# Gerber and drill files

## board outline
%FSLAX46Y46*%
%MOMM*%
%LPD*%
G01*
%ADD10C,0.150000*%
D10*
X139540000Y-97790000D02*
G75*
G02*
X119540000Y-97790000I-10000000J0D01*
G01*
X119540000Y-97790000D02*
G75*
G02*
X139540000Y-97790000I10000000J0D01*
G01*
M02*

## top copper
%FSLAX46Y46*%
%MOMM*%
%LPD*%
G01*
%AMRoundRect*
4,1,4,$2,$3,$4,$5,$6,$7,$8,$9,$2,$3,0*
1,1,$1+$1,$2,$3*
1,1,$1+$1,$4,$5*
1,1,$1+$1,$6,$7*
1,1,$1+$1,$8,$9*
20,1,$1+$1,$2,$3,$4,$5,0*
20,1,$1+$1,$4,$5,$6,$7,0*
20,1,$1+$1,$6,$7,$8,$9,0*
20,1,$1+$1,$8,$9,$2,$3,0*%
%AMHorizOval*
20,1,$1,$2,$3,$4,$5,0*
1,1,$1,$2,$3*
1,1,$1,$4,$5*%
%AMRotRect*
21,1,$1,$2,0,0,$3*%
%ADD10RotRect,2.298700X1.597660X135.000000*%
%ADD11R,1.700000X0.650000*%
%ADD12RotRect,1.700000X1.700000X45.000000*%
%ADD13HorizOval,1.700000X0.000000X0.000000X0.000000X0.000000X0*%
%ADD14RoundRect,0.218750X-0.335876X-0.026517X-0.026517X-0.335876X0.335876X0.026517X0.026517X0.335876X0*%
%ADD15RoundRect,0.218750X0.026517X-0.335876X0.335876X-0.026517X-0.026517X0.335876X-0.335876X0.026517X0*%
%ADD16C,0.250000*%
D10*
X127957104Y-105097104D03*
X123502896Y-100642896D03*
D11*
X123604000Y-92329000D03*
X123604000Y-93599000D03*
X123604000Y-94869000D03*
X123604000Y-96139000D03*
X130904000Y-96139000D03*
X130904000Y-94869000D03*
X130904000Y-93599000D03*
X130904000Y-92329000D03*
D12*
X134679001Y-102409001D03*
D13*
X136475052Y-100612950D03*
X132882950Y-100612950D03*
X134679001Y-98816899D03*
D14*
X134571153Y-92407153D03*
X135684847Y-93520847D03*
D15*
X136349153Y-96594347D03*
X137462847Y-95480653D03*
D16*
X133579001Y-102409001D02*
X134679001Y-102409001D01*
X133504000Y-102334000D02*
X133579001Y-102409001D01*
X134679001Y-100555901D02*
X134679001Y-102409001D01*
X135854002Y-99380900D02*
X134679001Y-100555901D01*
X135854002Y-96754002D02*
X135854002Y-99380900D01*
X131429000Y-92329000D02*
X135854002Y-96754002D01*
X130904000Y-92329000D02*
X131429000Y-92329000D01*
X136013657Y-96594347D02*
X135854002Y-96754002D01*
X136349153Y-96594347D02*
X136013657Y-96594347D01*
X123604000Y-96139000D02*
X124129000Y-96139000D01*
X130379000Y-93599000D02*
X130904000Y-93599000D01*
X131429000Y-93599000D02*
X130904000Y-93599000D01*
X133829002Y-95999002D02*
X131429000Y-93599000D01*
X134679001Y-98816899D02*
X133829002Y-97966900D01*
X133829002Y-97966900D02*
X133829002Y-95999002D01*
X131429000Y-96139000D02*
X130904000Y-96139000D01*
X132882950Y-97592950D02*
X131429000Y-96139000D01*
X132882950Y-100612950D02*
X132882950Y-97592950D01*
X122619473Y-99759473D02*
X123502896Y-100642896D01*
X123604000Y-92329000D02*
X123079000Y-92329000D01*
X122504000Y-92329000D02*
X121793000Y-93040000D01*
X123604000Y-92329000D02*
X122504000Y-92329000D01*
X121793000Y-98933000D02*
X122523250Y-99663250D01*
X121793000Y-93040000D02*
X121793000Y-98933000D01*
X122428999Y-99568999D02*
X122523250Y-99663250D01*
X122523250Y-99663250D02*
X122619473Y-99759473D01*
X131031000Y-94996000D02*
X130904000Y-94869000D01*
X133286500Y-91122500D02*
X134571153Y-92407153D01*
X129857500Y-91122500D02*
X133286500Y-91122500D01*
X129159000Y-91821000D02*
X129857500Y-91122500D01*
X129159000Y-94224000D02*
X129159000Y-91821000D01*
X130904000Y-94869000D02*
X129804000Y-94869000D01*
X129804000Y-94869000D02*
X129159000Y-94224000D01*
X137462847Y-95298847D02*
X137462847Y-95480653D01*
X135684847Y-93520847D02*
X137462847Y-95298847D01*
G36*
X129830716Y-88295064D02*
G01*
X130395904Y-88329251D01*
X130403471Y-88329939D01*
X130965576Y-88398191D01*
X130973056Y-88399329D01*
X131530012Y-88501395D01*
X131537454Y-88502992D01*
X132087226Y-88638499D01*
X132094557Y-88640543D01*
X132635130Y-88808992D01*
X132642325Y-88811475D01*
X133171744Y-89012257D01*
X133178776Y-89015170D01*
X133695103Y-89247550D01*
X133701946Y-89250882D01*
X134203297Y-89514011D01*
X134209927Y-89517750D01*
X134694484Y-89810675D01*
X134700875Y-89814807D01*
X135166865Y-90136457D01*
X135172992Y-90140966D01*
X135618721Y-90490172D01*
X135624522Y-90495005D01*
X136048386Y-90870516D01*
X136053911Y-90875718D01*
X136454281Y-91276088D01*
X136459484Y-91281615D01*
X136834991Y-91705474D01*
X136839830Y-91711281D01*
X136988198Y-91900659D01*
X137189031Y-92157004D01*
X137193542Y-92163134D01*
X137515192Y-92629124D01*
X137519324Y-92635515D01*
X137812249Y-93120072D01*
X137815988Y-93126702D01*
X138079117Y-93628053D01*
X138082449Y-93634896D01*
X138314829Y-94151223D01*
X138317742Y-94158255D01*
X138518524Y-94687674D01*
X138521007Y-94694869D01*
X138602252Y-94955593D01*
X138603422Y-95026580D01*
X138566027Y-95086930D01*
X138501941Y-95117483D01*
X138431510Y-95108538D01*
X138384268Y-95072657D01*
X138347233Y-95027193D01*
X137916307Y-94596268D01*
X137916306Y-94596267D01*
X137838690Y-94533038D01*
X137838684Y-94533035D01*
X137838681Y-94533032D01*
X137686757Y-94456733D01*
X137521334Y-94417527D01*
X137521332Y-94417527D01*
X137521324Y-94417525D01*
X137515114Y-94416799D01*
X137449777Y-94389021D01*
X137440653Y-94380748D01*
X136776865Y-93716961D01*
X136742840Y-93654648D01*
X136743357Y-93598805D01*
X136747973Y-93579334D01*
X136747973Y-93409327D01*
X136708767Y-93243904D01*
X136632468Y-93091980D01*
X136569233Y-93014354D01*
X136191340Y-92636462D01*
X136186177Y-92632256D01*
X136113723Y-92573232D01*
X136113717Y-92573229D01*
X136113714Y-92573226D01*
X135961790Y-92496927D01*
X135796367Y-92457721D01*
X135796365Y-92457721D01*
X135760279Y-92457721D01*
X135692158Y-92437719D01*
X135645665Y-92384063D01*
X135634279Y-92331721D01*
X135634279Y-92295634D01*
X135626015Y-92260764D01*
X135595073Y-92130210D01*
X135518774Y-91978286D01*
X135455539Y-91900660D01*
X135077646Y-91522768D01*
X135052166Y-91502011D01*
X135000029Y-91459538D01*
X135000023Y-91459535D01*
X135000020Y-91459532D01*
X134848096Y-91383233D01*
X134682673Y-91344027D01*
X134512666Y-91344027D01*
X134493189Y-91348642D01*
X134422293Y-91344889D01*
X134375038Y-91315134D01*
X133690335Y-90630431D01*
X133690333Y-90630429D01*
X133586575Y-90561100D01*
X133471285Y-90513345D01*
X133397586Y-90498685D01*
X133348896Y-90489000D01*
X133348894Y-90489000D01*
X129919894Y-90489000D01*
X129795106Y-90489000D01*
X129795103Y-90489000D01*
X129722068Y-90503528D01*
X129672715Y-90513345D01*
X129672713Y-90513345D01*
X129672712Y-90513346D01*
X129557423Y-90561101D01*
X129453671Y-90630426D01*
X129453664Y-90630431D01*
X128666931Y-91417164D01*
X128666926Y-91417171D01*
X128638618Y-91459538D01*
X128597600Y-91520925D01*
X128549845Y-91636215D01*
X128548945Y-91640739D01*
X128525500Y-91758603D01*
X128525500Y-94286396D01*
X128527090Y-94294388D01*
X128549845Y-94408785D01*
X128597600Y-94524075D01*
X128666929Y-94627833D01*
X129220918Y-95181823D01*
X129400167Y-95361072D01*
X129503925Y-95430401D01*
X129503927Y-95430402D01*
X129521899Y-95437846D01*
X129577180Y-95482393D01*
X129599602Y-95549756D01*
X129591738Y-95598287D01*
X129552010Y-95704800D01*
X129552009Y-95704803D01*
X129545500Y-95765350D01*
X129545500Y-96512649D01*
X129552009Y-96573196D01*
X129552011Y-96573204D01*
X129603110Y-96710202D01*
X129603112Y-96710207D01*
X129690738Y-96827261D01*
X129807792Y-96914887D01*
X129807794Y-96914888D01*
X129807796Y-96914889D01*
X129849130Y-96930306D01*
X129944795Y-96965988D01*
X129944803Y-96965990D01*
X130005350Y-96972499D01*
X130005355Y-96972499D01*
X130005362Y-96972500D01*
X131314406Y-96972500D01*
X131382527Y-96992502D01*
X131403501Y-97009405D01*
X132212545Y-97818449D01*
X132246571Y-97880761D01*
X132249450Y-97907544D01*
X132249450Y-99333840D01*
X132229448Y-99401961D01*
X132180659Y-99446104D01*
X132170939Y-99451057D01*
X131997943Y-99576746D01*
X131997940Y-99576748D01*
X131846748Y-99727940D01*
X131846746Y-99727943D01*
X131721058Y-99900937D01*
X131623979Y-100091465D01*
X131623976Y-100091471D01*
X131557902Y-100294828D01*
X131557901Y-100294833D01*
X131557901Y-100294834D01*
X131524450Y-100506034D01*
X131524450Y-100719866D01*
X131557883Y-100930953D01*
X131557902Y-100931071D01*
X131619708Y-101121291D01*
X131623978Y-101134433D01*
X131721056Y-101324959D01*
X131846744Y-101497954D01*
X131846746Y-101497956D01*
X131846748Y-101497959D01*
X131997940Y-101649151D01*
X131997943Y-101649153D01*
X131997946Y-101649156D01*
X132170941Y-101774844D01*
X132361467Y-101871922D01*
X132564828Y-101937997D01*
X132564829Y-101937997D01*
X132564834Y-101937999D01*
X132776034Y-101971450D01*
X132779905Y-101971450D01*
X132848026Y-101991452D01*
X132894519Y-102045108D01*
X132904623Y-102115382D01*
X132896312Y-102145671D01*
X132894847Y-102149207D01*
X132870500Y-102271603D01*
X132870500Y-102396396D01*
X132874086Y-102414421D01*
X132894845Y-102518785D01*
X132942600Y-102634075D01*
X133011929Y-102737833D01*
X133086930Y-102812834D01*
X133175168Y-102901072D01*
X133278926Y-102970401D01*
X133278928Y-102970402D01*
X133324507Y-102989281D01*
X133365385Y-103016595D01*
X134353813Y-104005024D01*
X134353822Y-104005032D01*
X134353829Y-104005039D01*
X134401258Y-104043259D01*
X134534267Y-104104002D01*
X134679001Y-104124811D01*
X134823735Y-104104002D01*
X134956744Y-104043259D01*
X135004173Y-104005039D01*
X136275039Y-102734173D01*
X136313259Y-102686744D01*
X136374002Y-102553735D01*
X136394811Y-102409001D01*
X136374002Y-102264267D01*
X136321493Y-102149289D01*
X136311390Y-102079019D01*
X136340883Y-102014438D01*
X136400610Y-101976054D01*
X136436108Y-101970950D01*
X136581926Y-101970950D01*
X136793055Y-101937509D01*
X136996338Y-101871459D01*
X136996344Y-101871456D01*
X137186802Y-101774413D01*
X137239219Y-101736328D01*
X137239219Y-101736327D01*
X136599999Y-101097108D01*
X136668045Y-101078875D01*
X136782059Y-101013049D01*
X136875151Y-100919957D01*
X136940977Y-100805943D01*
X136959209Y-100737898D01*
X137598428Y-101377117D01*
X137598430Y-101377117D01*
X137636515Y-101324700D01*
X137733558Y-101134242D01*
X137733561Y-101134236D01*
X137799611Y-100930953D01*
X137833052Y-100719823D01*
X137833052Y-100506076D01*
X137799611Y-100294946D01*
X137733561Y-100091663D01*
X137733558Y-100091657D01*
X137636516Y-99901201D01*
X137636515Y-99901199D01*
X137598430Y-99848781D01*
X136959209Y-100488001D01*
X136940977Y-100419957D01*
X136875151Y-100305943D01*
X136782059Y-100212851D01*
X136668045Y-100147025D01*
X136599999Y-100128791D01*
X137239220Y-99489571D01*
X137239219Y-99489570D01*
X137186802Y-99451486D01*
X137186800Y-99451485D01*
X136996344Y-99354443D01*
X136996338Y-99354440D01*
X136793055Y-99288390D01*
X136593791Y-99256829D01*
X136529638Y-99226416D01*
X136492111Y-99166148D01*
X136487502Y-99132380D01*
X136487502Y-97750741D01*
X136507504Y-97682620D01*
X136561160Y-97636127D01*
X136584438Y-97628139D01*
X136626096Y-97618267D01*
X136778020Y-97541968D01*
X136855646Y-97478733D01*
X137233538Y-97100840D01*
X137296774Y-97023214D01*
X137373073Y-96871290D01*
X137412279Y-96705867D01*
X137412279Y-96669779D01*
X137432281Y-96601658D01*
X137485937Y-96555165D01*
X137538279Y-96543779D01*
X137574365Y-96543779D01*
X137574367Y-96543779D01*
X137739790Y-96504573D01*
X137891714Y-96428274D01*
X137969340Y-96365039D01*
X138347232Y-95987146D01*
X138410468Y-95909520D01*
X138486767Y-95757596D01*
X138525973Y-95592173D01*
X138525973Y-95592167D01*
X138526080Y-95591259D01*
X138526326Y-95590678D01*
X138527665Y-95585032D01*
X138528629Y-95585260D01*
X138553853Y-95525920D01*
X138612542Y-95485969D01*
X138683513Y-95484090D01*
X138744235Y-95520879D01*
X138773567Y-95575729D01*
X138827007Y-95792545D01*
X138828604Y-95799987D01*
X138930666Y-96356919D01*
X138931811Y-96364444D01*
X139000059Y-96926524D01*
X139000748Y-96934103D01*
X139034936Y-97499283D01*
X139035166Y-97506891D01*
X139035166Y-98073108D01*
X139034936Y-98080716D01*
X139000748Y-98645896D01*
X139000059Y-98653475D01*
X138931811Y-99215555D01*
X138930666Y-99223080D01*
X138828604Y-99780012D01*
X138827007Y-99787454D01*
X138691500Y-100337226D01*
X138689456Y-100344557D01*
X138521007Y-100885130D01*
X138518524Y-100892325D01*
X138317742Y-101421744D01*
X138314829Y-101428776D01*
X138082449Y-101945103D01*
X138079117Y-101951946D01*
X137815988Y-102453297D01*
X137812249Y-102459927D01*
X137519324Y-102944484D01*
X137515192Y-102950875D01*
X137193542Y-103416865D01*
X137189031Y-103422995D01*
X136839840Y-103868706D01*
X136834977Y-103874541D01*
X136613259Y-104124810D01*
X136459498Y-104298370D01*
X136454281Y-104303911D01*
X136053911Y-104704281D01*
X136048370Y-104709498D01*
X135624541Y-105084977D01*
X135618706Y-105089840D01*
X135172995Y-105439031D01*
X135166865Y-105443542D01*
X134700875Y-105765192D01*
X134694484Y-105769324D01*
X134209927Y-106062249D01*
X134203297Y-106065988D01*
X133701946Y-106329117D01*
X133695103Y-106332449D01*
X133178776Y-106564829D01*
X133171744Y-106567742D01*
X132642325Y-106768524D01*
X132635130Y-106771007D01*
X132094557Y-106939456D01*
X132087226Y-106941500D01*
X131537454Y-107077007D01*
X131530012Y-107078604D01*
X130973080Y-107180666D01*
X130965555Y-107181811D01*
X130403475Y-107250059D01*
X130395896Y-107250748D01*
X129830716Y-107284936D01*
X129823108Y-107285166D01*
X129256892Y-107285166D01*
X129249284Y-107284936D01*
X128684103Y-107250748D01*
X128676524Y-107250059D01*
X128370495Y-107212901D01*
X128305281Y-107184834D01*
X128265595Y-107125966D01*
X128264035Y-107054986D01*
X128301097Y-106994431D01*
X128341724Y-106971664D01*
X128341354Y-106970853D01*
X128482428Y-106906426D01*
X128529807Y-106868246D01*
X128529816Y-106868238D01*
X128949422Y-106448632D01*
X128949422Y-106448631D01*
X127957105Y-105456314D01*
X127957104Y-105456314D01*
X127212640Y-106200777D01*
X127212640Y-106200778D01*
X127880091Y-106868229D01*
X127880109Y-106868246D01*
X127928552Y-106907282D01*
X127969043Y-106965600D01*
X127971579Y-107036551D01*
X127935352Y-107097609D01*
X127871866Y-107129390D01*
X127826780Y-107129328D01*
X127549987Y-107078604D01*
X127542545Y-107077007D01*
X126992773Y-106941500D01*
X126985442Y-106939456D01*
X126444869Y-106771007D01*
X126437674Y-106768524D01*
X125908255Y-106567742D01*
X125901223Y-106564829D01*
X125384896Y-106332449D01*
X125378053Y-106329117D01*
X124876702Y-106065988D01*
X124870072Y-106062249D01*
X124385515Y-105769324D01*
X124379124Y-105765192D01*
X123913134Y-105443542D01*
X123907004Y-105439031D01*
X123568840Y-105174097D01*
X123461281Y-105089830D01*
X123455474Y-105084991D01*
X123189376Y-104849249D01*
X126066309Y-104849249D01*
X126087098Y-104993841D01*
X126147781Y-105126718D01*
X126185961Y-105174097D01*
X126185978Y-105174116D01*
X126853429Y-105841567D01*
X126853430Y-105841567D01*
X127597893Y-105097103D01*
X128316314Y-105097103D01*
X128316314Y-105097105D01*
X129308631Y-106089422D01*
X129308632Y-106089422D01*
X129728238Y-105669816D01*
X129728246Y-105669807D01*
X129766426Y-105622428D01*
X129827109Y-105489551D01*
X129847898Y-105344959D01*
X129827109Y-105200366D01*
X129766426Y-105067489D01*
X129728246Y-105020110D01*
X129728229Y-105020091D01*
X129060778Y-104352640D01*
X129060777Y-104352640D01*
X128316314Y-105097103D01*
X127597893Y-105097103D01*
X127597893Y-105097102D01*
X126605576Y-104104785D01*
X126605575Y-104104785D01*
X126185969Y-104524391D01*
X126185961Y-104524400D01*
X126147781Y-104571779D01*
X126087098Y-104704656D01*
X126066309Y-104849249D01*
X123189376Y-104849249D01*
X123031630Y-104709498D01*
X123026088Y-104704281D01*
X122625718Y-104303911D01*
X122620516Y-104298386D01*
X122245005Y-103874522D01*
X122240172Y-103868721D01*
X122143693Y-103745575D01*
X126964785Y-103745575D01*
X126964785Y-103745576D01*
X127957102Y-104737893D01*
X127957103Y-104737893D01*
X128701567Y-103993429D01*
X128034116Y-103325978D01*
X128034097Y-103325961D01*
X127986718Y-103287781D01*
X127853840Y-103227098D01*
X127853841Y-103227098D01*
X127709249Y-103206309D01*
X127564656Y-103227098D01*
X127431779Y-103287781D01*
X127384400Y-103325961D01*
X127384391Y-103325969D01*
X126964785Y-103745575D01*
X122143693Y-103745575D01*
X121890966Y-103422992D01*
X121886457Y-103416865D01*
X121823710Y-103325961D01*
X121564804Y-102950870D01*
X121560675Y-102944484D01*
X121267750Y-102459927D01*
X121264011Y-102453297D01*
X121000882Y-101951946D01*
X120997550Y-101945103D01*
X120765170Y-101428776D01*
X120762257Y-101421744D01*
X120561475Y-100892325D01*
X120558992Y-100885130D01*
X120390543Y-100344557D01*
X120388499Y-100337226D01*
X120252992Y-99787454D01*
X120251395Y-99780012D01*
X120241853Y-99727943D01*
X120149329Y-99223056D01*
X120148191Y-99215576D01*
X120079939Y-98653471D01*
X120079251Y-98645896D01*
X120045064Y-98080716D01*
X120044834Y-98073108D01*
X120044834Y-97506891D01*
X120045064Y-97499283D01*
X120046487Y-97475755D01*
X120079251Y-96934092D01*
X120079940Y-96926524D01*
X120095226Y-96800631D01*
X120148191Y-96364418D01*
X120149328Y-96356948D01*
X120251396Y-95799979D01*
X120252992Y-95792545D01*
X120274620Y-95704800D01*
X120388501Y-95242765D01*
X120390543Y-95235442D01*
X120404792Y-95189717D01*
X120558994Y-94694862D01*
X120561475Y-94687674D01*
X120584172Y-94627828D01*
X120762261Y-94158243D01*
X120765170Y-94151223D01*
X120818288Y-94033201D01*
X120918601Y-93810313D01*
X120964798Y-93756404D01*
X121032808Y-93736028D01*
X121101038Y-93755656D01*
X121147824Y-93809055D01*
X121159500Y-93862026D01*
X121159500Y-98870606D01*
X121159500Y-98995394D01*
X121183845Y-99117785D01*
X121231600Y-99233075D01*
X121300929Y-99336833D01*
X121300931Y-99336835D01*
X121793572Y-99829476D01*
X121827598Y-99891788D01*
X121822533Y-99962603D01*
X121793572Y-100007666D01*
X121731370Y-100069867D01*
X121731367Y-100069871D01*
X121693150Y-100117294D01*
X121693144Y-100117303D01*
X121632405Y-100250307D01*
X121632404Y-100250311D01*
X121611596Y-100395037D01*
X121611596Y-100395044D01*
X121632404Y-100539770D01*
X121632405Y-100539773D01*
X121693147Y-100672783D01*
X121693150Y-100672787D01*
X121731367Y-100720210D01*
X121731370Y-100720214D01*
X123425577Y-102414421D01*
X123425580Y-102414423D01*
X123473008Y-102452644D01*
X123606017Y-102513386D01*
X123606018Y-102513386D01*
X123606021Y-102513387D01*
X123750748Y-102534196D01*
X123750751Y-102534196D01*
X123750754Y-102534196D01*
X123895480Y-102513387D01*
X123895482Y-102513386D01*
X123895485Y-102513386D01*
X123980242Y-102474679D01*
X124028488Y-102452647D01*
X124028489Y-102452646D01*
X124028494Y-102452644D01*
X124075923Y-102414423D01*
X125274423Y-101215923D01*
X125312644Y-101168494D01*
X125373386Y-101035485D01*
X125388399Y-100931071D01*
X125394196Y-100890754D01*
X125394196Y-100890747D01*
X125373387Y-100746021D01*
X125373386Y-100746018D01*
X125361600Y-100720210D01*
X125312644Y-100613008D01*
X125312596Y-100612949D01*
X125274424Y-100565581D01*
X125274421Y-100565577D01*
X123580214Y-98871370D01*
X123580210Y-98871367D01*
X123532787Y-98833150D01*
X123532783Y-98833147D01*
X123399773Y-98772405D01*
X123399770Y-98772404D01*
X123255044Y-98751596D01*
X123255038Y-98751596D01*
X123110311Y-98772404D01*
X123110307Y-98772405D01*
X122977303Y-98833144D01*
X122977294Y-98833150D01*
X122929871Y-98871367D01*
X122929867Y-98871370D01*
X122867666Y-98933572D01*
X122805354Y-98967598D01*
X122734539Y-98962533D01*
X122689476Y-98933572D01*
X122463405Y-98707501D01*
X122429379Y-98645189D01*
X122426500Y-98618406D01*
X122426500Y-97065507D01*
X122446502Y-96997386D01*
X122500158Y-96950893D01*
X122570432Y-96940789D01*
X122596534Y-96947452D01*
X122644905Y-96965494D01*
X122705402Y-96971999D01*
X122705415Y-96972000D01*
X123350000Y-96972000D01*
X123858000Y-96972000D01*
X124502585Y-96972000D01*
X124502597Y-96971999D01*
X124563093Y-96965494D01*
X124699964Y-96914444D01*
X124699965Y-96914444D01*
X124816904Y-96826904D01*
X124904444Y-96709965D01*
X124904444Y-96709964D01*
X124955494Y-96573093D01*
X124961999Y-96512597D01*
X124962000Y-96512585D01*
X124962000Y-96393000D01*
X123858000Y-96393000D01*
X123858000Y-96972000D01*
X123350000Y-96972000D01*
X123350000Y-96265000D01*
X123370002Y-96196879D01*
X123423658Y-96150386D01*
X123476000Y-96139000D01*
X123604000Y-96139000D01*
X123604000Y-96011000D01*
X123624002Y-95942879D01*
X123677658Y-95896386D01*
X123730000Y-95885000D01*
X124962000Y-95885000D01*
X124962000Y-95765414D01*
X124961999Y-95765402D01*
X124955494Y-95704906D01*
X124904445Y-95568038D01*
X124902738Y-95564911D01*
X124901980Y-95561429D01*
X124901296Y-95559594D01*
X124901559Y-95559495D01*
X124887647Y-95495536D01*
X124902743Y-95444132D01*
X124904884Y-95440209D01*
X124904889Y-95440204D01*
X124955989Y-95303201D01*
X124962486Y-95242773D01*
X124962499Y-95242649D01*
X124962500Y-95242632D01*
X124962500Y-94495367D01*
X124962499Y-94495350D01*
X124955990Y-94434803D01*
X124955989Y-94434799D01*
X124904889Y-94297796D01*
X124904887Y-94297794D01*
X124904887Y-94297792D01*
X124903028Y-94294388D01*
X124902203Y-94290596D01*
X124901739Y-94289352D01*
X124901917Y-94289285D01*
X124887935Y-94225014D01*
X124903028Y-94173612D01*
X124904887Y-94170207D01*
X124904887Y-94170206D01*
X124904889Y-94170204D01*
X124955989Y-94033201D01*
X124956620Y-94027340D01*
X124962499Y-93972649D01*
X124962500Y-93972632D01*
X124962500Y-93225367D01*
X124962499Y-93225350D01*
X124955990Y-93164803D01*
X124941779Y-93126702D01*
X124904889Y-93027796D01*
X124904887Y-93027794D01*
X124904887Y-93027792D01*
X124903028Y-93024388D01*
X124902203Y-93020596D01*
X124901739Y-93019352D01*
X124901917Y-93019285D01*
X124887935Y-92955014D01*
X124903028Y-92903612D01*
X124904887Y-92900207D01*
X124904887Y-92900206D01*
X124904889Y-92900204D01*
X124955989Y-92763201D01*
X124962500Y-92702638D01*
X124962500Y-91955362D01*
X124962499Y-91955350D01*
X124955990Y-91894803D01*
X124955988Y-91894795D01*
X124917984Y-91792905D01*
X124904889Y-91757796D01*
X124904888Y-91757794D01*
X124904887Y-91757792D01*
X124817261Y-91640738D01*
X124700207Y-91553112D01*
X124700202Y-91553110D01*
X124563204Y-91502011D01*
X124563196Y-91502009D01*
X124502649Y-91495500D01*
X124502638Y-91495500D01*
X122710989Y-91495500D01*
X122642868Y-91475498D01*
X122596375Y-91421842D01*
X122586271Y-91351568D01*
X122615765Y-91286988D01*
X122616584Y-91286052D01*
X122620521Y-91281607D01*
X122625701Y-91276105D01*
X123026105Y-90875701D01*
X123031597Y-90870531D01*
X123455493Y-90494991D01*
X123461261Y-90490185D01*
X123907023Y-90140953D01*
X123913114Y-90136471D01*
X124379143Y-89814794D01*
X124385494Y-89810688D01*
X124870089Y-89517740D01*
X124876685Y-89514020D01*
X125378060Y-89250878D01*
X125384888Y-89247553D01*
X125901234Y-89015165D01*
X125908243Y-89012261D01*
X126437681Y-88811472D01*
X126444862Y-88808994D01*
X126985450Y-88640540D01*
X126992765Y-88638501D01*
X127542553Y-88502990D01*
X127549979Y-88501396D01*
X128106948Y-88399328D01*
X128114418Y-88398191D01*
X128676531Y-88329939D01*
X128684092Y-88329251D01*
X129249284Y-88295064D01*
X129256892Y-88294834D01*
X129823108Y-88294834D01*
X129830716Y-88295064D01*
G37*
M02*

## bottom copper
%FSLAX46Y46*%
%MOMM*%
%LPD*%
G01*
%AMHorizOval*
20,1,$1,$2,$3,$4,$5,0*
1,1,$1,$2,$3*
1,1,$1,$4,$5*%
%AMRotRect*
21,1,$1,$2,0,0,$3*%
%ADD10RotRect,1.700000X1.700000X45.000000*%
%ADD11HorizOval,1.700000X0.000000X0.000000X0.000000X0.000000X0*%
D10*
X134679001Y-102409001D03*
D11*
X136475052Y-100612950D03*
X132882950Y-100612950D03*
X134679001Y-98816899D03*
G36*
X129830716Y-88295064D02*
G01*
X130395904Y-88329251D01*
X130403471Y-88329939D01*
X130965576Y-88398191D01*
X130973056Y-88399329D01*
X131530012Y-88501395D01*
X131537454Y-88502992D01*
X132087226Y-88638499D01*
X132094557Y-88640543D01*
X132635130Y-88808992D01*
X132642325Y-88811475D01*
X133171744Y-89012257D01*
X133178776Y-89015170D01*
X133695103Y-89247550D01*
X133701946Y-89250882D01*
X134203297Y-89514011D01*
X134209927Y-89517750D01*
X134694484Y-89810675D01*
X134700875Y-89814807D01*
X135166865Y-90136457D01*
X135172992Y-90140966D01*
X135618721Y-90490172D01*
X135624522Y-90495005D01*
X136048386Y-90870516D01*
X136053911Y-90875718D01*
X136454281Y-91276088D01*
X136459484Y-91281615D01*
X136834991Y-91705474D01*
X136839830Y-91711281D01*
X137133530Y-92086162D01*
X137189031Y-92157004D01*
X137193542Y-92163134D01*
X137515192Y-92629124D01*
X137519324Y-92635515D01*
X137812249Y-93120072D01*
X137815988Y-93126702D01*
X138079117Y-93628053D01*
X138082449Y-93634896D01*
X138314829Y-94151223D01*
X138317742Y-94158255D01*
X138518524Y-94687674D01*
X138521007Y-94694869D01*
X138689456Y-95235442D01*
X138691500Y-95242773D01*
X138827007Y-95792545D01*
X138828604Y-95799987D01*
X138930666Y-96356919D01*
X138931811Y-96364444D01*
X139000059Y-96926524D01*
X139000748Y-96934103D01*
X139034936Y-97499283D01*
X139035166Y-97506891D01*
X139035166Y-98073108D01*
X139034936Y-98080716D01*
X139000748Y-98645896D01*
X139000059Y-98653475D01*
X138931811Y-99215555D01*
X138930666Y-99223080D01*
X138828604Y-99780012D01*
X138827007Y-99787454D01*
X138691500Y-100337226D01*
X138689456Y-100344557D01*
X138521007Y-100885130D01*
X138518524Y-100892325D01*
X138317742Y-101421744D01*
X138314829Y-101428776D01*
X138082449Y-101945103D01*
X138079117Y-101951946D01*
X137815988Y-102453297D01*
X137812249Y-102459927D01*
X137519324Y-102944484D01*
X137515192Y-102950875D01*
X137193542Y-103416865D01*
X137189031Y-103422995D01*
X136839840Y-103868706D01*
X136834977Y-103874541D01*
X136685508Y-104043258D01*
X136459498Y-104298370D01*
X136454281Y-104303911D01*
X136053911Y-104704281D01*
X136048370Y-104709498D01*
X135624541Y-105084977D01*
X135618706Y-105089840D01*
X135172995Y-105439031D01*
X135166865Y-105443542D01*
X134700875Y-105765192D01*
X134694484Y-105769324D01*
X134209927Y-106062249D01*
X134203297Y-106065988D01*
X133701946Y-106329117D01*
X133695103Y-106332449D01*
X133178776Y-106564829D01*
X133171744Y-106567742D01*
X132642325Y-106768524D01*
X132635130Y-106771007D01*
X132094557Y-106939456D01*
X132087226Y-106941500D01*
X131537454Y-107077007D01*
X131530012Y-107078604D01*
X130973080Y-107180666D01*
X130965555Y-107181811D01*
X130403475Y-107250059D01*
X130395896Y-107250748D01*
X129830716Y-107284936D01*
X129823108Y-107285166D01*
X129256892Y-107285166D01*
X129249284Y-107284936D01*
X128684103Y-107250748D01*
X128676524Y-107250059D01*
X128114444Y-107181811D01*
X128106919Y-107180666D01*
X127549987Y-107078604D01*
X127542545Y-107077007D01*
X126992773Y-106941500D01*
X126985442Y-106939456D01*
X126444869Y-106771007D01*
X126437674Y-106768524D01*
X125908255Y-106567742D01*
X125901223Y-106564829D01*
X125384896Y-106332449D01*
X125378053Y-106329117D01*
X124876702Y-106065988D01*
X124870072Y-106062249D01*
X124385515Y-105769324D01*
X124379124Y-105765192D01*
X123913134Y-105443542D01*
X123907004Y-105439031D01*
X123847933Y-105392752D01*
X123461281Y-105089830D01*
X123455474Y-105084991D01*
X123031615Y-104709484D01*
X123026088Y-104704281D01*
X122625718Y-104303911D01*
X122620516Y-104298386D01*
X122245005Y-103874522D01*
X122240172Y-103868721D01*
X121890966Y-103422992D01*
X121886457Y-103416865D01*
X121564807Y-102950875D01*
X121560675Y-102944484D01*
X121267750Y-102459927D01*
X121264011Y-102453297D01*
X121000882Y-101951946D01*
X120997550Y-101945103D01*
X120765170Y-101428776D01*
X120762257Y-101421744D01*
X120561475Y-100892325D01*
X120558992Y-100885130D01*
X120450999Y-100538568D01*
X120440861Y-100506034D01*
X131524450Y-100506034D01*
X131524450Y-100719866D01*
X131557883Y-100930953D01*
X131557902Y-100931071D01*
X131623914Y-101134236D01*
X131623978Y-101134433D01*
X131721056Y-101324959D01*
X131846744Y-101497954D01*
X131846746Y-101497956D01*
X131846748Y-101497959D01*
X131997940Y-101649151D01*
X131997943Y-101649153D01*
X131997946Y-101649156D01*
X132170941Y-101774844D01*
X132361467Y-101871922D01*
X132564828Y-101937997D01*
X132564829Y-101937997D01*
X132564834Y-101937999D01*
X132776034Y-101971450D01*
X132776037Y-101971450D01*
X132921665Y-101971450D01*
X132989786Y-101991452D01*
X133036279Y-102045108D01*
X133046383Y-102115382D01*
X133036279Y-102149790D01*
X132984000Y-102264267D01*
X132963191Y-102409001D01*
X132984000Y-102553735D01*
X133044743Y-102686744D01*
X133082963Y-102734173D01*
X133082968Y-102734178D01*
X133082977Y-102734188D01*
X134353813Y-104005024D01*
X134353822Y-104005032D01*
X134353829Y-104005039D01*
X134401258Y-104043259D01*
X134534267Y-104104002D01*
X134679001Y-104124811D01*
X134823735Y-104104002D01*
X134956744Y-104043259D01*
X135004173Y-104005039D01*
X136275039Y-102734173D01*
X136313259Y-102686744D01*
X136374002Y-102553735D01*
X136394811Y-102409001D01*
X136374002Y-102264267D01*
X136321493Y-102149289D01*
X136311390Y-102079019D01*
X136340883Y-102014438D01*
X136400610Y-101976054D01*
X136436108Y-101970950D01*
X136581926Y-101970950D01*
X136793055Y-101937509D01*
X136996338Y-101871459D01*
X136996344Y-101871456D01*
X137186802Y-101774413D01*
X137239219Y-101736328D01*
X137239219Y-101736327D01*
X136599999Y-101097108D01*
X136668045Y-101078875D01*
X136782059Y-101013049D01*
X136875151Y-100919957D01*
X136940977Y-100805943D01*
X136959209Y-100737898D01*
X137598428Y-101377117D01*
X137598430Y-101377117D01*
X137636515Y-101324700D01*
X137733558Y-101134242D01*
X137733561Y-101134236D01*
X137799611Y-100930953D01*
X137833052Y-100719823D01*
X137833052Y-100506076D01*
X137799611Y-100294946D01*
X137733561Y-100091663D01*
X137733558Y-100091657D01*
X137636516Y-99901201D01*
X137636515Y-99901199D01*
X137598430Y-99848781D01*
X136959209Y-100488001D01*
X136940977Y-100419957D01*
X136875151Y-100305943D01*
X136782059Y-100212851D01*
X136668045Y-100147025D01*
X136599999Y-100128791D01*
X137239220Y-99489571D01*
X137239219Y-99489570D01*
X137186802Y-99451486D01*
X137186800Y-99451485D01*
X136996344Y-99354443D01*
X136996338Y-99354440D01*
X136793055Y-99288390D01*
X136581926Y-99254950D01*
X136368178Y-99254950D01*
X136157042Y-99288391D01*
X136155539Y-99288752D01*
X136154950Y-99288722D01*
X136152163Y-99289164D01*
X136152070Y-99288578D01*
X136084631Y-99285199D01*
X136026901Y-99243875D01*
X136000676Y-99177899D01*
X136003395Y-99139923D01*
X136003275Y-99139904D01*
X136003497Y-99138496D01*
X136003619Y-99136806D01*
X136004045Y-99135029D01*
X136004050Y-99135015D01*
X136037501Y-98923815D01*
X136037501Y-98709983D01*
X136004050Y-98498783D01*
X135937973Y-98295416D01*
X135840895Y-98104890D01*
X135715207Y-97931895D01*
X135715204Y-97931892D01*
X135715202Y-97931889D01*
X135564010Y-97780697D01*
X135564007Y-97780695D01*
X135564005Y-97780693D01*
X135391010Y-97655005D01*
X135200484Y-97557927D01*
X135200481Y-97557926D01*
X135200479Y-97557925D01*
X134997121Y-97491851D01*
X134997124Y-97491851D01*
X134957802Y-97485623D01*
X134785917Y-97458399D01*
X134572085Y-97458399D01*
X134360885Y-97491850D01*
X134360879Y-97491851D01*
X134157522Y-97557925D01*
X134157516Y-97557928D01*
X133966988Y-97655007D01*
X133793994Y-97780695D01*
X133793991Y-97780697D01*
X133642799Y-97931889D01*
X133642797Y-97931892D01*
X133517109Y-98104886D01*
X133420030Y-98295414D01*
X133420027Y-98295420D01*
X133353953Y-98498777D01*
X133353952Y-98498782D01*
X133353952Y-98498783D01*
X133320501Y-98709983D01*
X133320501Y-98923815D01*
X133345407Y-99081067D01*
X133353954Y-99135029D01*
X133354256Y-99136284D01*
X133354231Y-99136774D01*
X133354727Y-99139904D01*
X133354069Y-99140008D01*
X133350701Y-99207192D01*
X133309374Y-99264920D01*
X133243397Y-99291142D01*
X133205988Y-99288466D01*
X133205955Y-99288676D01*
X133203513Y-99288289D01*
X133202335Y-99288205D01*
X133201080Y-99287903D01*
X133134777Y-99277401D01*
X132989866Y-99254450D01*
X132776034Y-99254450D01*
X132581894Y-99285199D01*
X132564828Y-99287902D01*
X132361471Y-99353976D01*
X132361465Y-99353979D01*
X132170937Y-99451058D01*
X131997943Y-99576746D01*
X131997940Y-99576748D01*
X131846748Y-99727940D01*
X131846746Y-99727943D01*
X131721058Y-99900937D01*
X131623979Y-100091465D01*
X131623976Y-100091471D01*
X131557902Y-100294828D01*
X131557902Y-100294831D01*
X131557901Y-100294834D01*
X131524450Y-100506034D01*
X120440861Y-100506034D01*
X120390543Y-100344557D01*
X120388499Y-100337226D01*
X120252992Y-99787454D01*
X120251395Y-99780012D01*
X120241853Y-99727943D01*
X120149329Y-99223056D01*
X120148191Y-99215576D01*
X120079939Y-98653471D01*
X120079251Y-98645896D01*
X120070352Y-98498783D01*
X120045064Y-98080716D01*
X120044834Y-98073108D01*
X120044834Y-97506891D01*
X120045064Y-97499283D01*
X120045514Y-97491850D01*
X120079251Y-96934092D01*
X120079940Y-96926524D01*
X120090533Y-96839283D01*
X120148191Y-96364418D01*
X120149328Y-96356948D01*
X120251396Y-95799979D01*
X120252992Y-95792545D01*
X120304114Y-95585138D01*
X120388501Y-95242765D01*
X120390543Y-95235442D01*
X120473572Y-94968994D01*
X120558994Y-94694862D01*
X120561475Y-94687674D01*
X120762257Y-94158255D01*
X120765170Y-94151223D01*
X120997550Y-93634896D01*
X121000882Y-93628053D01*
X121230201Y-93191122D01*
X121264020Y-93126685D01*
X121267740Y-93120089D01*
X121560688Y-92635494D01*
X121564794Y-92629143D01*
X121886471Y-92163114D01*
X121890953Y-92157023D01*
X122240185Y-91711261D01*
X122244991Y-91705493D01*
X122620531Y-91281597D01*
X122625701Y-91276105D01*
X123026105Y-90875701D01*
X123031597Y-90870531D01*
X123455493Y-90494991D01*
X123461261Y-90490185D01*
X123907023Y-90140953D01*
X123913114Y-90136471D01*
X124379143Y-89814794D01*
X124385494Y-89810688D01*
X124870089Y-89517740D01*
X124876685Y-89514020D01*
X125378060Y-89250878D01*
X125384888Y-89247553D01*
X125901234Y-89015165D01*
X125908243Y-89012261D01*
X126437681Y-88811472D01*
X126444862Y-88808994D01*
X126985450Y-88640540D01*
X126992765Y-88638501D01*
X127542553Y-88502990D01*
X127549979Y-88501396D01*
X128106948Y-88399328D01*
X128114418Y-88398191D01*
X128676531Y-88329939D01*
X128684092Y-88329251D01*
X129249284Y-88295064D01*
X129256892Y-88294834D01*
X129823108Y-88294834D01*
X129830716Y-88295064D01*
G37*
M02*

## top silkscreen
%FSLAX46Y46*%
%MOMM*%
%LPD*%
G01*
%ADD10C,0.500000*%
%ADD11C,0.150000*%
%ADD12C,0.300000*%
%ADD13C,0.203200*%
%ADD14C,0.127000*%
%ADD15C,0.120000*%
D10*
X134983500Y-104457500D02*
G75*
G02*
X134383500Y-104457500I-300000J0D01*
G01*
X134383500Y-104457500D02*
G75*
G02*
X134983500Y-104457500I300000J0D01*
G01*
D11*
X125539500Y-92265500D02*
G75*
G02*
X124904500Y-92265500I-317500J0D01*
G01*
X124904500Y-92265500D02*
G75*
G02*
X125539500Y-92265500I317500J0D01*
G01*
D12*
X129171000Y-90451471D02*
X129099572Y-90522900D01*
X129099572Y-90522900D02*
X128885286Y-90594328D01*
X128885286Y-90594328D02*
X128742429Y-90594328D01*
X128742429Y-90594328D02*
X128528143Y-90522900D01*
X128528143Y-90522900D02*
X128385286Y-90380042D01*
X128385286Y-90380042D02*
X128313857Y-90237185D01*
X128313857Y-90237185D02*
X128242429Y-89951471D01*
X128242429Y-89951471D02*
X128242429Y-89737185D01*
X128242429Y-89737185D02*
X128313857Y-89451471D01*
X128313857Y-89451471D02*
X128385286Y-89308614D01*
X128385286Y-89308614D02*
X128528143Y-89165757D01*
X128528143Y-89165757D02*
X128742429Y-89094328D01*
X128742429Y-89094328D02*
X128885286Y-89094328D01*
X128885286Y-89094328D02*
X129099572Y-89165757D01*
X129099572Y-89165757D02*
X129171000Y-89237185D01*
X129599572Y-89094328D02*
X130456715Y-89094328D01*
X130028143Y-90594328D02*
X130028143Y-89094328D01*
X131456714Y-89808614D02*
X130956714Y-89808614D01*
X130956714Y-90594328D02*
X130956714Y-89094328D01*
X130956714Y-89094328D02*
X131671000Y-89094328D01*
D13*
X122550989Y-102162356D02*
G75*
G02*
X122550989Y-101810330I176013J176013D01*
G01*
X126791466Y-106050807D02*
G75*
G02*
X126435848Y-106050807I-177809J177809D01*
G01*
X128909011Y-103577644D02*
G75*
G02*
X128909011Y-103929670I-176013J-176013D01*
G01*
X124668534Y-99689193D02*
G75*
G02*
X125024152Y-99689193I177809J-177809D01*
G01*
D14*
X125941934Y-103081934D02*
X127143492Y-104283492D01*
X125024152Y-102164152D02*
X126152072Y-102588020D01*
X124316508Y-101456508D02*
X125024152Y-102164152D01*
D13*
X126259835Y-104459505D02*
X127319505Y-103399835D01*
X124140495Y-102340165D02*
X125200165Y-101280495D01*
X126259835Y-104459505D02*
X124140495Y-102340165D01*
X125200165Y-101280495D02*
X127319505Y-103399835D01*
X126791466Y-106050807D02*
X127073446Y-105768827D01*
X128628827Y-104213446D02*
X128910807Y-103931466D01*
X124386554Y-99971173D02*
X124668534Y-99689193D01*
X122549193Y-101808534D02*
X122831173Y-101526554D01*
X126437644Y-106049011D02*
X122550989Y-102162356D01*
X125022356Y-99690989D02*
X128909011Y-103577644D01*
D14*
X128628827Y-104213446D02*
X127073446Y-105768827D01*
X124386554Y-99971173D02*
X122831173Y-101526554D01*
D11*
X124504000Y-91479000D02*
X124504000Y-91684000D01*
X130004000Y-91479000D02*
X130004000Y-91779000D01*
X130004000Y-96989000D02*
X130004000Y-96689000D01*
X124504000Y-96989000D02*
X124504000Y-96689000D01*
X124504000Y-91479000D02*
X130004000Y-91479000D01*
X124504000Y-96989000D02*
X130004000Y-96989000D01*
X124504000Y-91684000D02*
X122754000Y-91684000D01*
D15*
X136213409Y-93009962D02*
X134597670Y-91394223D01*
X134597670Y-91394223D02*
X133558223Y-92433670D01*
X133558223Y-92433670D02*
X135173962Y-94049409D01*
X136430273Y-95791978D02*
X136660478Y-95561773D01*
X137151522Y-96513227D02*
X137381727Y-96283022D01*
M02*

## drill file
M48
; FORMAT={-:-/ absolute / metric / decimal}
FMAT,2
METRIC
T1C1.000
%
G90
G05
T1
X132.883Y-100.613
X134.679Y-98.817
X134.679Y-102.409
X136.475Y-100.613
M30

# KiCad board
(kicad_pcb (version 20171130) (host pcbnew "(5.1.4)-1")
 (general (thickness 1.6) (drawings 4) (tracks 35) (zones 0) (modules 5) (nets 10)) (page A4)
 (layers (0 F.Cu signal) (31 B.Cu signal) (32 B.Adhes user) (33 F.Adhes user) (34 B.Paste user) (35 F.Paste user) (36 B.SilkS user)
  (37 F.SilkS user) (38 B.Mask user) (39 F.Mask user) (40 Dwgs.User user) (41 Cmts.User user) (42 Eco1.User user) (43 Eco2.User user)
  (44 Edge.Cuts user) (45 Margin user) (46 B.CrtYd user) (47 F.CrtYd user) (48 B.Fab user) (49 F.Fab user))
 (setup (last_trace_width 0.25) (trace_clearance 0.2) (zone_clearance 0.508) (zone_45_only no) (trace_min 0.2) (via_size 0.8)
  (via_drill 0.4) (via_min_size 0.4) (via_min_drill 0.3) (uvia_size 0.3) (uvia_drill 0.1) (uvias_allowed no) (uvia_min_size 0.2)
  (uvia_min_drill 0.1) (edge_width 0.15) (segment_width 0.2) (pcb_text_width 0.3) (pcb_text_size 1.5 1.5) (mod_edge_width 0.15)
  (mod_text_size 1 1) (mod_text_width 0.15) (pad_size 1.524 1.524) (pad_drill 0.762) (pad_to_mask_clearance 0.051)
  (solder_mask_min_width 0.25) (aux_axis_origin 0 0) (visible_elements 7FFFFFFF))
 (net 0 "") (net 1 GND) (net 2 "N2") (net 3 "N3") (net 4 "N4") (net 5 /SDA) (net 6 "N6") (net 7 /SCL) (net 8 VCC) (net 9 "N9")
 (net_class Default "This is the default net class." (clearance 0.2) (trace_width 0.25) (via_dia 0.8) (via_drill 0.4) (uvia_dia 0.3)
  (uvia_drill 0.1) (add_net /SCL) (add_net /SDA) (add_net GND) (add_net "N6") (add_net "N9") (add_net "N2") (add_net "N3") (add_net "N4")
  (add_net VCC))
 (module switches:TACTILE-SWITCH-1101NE (layer F.Cu) (at 125.73 102.87 315)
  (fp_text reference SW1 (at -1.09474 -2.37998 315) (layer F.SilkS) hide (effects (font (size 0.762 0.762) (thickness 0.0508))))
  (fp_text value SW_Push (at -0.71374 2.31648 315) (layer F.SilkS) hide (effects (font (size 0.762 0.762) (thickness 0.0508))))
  (fp_arc (start -2.74828 1.4986) (end -2.74828 1.74752) (angle 90) (layer F.SilkS) (width 0.2032))
  (fp_arc (start 2.74828 1.4986) (end 2.99974 1.4986) (angle 90) (layer F.SilkS) (width 0.2032))
  (fp_arc (start 2.74828 -1.4986) (end 2.74828 -1.74752) (angle 90) (layer F.SilkS) (width 0.2032))
  (fp_arc (start -2.74828 -1.4986) (end -2.99974 -1.4986) (angle 90) (layer F.SilkS) (width 0.2032))
  (fp_line (start 0.29972 0) (end 1.99898 0) (layer F.SilkS) (width 0.127))
  (fp_line (start -0.99822 0) (end 0.09906 -0.49784) (layer F.SilkS) (width 0.127))
  (fp_line (start -1.99898 0) (end -0.99822 0) (layer F.SilkS) (width 0.127))
  (fp_line (start 1.4986 0.7493) (end 1.4986 -0.7493) (layer F.SilkS) (width 0.2032))
  (fp_line (start -1.4986 0.7493) (end -1.4986 -0.7493) (layer F.SilkS) (width 0.2032))
  (fp_line (start 1.4986 0.7493) (end -1.4986 0.7493) (layer F.SilkS) (width 0.2032))
  (fp_line (start -1.4986 -0.7493) (end 1.4986 -0.7493) (layer F.SilkS) (width 0.2032))
  (fp_line (start 2.99974 1.4986) (end 2.99974 1.09982) (layer F.SilkS) (width 0.2032))
  (fp_line (start 2.99974 -1.09982) (end 2.99974 -1.4986) (layer F.SilkS) (width 0.2032))
  (fp_line (start -2.99974 -1.09982) (end -2.99974 -1.4986) (layer F.SilkS) (width 0.2032))
  (fp_line (start -2.99974 1.4986) (end -2.99974 1.09982) (layer F.SilkS) (width 0.2032))
  (fp_line (start 2.74828 1.74752) (end -2.74828 1.74752) (layer F.SilkS) (width 0.2032))
  (fp_line (start -2.74828 -1.74752) (end 2.74828 -1.74752) (layer F.SilkS) (width 0.2032))
  (fp_line (start 2.99974 -1.09982) (end 2.99974 1.09982) (layer F.SilkS) (width 0.127))
  (fp_line (start -2.99974 -1.09982) (end -2.99974 1.09982) (layer F.SilkS) (width 0.127))
  (pad 2 smd rect (at 3.149601 0 135) (size 2.2987 1.59766) (layers F.Cu F.Paste F.Mask) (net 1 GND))
  (pad 1 smd rect (at -3.149601 0 135) (size 2.2987 1.59766) (layers F.Cu F.Paste F.Mask) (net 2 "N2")))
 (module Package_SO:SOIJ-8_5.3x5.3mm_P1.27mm (layer F.Cu) (at 127.254 94.234)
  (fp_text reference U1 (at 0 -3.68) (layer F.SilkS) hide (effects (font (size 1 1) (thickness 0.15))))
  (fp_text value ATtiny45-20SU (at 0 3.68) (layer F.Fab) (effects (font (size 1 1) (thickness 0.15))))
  (fp_line (start -2.75 -2.755) (end -2.75 -2.55) (layer F.SilkS) (width 0.15))
  (fp_line (start 2.75 -2.755) (end 2.75 -2.455) (layer F.SilkS) (width 0.15))
  (fp_line (start 2.75 2.755) (end 2.75 2.455) (layer F.SilkS) (width 0.15))
  (fp_line (start -2.75 2.755) (end -2.75 2.455) (layer F.SilkS) (width 0.15))
  (fp_line (start -2.75 -2.755) (end 2.75 -2.755) (layer F.SilkS) (width 0.15))
  (fp_line (start -2.75 2.755) (end 2.75 2.755) (layer F.SilkS) (width 0.15))
  (fp_line (start -2.75 -2.55) (end -4.5 -2.55) (layer F.SilkS) (width 0.15))
  (pad 1 smd rect (at -3.65 -1.905) (size 1.7 0.65) (layers F.Cu F.Paste F.Mask) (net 2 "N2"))
  (pad 2 smd rect (at -3.65 -0.635) (size 1.7 0.65) (layers F.Cu F.Paste F.Mask) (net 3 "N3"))
  (pad 3 smd rect (at -3.65 0.635) (size 1.7 0.65) (layers F.Cu F.Paste F.Mask) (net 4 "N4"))
  (pad 4 smd rect (at -3.65 1.905) (size 1.7 0.65) (layers F.Cu F.Paste F.Mask) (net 1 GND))
  (pad 5 smd rect (at 3.65 1.905) (size 1.7 0.65) (layers F.Cu F.Paste F.Mask) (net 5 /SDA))
  (pad 6 smd rect (at 3.65 0.635) (size 1.7 0.65) (layers F.Cu F.Paste F.Mask) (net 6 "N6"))
  (pad 7 smd rect (at 3.65 -0.635) (size 1.7 0.65) (layers F.Cu F.Paste F.Mask) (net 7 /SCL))
  (pad 8 smd rect (at 3.65 -1.905) (size 1.7 0.65) (layers F.Cu F.Paste F.Mask) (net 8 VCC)))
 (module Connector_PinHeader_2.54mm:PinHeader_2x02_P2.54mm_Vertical (layer B.Cu) (at 134.679001 102.409001 45)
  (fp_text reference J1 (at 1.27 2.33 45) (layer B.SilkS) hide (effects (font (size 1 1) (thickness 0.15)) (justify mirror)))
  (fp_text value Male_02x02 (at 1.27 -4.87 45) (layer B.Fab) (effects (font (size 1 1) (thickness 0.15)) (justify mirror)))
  (pad 1 thru_hole rect (at 0 0 45) (size 1.7 1.7) (drill 1) (layers *.Cu *.Mask) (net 8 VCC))
  (pad 2 thru_hole oval (at 2.54 0 45) (size 1.7 1.7) (drill 1) (layers *.Cu *.Mask) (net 1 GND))
  (pad 3 thru_hole oval (at 0 -2.54 45) (size 1.7 1.7) (drill 1) (layers *.Cu *.Mask) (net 5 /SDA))
  (pad 4 thru_hole oval (at 2.54 -2.54 45) (size 1.7 1.7) (drill 1) (layers *.Cu *.Mask) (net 7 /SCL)))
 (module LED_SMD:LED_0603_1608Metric (layer F.Cu) (at 135.128 92.964 315)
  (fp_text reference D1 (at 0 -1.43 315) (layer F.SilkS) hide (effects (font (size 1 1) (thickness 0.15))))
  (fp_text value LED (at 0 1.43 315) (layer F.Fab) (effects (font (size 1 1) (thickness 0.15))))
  (fp_line (start 0.8 -0.735) (end -1.485 -0.735) (layer F.SilkS) (width 0.12))
  (fp_line (start -1.485 -0.735) (end -1.485 0.735) (layer F.SilkS) (width 0.12))
  (fp_line (start -1.485 0.735) (end 0.8 0.735) (layer F.SilkS) (width 0.12))
  (pad 1 smd roundrect (at -0.787501 0 315) (size 0.875 0.95) (layers F.Cu F.Paste F.Mask) (roundrect_rratio 0.25) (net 6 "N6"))
  (pad 2 smd roundrect (at 0.787501 0 315) (size 0.875 0.95) (layers F.Cu F.Paste F.Mask) (roundrect_rratio 0.25) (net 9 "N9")))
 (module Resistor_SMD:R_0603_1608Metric (layer F.Cu) (at 136.906 96.0375 45)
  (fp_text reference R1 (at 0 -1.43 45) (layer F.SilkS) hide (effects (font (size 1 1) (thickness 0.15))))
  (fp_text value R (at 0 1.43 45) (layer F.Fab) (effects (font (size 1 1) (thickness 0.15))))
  (fp_line (start -0.162779 -0.51) (end 0.162779 -0.51) (layer F.SilkS) (width 0.12))
  (fp_line (start -0.162779 0.51) (end 0.162779 0.51) (layer F.SilkS) (width 0.12))
  (pad 1 smd roundrect (at -0.7875 0 45) (size 0.875 0.95) (layers F.Cu F.Paste F.Mask) (roundrect_rratio 0.25) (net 8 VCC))
  (pad 2 smd roundrect (at 0.7875 0 45) (size 0.875 0.95) (layers F.Cu F.Paste F.Mask) (roundrect_rratio 0.25) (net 9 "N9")))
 (gr_circle (center 134.6835 104.4575) (end 134.9835 104.4575) (layer F.SilkS) (width 0.5))
 (gr_circle (center 125.222 92.2655) (end 125.476 92.456) (layer F.SilkS) (width 0.15))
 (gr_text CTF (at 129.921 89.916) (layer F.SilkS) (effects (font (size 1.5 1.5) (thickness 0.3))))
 (gr_circle (center 129.54 97.79) (end 139.54 97.79) (layer Edge.Cuts) (width 0.15))
 (segment (start 133.579001 102.409001) (end 134.679001 102.409001) (width 0.25) (layer F.Cu) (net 8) (status 30))
 (segment (start 133.504 102.334) (end 133.579001 102.409001) (width 0.25) (layer F.Cu) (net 8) (status 20))
 (segment (start 134.679001 100.555901) (end 134.679001 102.409001) (width 0.25) (layer F.Cu) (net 8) (status 20))
 (segment (start 135.854002 99.3809) (end 134.679001 100.555901) (width 0.25) (layer F.Cu) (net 8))
 (segment (start 135.854002 96.754002) (end 135.854002 99.3809) (width 0.25) (layer F.Cu) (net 8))
 (segment (start 131.429 92.329) (end 135.854002 96.754002) (width 0.25) (layer F.Cu) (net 8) (status 10))
 (segment (start 130.904 92.329) (end 131.429 92.329) (width 0.25) (layer F.Cu) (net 8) (status 30))
 (segment (start 136.013657 96.594347) (end 135.854002 96.754002) (width 0.25) (layer F.Cu) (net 8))
 (segment (start 136.349153 96.594347) (end 136.013657 96.594347) (width 0.25) (layer F.Cu) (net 8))
 (segment (start 123.604 96.139) (end 124.129 96.139) (width 0.25) (layer F.Cu) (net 1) (status 30))
 (segment (start 130.379 93.599) (end 130.904 93.599) (width 0.25) (layer F.Cu) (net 7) (status 30))
 (segment (start 131.429 93.599) (end 130.904 93.599) (width 0.25) (layer F.Cu) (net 7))
 (segment (start 133.829002 95.999002) (end 131.429 93.599) (width 0.25) (layer F.Cu) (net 7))
 (segment (start 134.679001 98.816899) (end 133.829002 97.9669) (width 0.25) (layer F.Cu) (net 7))
 (segment (start 133.829002 97.9669) (end 133.829002 95.999002) (width 0.25) (layer F.Cu) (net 7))
 (segment (start 131.429 96.139) (end 130.904 96.139) (width 0.25) (layer F.Cu) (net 5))
 (segment (start 132.88295 97.59295) (end 131.429 96.139) (width 0.25) (layer F.Cu) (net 5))
 (segment (start 132.88295 100.61295) (end 132.88295 97.59295) (width 0.25) (layer F.Cu) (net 5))
 (segment (start 122.619473 99.759473) (end 123.502896 100.642896) (width 0.25) (layer F.Cu) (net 2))
 (segment (start 123.604 92.329) (end 123.079 92.329) (width 0.25) (layer F.Cu) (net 2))
 (segment (start 122.504 92.329) (end 121.793 93.04) (width 0.25) (layer F.Cu) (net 2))
 (segment (start 123.604 92.329) (end 122.504 92.329) (width 0.25) (layer F.Cu) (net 2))
 (segment (start 121.793 98.933) (end 122.52325 99.66325) (width 0.25) (layer F.Cu) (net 2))
 (segment (start 121.793 93.04) (end 121.793 98.933) (width 0.25) (layer F.Cu) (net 2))
 (segment (start 122.428999 99.568999) (end 122.52325 99.66325) (width 0.25) (layer F.Cu) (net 2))
 (segment (start 122.52325 99.66325) (end 122.619473 99.759473) (width 0.25) (layer F.Cu) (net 2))
 (segment (start 131.031 94.996) (end 130.904 94.869) (width 0.25) (layer F.Cu) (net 6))
 (segment (start 133.2865 91.1225) (end 134.571153 92.407153) (width 0.25) (layer F.Cu) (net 6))
 (segment (start 129.8575 91.1225) (end 133.2865 91.1225) (width 0.25) (layer F.Cu) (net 6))
 (segment (start 129.159 91.821) (end 129.8575 91.1225) (width 0.25) (layer F.Cu) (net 6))
 (segment (start 129.159 94.224) (end 129.159 91.821) (width 0.25) (layer F.Cu) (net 6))
 (segment (start 130.904 94.869) (end 129.804 94.869) (width 0.25) (layer F.Cu) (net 6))
 (segment (start 129.804 94.869) (end 129.159 94.224) (width 0.25) (layer F.Cu) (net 6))
 (segment (start 137.462847 95.298847) (end 137.462847 95.480653) (width 0.25) (layer F.Cu) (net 9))
 (segment (start 135.684847 93.520847) (end 137.462847 95.298847) (width 0.25) (layer F.Cu) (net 9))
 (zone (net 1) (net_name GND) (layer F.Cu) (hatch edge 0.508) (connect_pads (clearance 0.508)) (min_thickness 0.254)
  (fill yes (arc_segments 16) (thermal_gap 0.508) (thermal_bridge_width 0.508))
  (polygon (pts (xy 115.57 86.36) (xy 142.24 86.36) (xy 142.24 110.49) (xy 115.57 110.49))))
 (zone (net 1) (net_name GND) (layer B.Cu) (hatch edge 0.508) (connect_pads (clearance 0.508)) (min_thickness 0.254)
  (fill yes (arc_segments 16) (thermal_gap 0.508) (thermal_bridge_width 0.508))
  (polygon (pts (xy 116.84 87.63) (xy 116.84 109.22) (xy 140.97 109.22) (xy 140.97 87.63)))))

